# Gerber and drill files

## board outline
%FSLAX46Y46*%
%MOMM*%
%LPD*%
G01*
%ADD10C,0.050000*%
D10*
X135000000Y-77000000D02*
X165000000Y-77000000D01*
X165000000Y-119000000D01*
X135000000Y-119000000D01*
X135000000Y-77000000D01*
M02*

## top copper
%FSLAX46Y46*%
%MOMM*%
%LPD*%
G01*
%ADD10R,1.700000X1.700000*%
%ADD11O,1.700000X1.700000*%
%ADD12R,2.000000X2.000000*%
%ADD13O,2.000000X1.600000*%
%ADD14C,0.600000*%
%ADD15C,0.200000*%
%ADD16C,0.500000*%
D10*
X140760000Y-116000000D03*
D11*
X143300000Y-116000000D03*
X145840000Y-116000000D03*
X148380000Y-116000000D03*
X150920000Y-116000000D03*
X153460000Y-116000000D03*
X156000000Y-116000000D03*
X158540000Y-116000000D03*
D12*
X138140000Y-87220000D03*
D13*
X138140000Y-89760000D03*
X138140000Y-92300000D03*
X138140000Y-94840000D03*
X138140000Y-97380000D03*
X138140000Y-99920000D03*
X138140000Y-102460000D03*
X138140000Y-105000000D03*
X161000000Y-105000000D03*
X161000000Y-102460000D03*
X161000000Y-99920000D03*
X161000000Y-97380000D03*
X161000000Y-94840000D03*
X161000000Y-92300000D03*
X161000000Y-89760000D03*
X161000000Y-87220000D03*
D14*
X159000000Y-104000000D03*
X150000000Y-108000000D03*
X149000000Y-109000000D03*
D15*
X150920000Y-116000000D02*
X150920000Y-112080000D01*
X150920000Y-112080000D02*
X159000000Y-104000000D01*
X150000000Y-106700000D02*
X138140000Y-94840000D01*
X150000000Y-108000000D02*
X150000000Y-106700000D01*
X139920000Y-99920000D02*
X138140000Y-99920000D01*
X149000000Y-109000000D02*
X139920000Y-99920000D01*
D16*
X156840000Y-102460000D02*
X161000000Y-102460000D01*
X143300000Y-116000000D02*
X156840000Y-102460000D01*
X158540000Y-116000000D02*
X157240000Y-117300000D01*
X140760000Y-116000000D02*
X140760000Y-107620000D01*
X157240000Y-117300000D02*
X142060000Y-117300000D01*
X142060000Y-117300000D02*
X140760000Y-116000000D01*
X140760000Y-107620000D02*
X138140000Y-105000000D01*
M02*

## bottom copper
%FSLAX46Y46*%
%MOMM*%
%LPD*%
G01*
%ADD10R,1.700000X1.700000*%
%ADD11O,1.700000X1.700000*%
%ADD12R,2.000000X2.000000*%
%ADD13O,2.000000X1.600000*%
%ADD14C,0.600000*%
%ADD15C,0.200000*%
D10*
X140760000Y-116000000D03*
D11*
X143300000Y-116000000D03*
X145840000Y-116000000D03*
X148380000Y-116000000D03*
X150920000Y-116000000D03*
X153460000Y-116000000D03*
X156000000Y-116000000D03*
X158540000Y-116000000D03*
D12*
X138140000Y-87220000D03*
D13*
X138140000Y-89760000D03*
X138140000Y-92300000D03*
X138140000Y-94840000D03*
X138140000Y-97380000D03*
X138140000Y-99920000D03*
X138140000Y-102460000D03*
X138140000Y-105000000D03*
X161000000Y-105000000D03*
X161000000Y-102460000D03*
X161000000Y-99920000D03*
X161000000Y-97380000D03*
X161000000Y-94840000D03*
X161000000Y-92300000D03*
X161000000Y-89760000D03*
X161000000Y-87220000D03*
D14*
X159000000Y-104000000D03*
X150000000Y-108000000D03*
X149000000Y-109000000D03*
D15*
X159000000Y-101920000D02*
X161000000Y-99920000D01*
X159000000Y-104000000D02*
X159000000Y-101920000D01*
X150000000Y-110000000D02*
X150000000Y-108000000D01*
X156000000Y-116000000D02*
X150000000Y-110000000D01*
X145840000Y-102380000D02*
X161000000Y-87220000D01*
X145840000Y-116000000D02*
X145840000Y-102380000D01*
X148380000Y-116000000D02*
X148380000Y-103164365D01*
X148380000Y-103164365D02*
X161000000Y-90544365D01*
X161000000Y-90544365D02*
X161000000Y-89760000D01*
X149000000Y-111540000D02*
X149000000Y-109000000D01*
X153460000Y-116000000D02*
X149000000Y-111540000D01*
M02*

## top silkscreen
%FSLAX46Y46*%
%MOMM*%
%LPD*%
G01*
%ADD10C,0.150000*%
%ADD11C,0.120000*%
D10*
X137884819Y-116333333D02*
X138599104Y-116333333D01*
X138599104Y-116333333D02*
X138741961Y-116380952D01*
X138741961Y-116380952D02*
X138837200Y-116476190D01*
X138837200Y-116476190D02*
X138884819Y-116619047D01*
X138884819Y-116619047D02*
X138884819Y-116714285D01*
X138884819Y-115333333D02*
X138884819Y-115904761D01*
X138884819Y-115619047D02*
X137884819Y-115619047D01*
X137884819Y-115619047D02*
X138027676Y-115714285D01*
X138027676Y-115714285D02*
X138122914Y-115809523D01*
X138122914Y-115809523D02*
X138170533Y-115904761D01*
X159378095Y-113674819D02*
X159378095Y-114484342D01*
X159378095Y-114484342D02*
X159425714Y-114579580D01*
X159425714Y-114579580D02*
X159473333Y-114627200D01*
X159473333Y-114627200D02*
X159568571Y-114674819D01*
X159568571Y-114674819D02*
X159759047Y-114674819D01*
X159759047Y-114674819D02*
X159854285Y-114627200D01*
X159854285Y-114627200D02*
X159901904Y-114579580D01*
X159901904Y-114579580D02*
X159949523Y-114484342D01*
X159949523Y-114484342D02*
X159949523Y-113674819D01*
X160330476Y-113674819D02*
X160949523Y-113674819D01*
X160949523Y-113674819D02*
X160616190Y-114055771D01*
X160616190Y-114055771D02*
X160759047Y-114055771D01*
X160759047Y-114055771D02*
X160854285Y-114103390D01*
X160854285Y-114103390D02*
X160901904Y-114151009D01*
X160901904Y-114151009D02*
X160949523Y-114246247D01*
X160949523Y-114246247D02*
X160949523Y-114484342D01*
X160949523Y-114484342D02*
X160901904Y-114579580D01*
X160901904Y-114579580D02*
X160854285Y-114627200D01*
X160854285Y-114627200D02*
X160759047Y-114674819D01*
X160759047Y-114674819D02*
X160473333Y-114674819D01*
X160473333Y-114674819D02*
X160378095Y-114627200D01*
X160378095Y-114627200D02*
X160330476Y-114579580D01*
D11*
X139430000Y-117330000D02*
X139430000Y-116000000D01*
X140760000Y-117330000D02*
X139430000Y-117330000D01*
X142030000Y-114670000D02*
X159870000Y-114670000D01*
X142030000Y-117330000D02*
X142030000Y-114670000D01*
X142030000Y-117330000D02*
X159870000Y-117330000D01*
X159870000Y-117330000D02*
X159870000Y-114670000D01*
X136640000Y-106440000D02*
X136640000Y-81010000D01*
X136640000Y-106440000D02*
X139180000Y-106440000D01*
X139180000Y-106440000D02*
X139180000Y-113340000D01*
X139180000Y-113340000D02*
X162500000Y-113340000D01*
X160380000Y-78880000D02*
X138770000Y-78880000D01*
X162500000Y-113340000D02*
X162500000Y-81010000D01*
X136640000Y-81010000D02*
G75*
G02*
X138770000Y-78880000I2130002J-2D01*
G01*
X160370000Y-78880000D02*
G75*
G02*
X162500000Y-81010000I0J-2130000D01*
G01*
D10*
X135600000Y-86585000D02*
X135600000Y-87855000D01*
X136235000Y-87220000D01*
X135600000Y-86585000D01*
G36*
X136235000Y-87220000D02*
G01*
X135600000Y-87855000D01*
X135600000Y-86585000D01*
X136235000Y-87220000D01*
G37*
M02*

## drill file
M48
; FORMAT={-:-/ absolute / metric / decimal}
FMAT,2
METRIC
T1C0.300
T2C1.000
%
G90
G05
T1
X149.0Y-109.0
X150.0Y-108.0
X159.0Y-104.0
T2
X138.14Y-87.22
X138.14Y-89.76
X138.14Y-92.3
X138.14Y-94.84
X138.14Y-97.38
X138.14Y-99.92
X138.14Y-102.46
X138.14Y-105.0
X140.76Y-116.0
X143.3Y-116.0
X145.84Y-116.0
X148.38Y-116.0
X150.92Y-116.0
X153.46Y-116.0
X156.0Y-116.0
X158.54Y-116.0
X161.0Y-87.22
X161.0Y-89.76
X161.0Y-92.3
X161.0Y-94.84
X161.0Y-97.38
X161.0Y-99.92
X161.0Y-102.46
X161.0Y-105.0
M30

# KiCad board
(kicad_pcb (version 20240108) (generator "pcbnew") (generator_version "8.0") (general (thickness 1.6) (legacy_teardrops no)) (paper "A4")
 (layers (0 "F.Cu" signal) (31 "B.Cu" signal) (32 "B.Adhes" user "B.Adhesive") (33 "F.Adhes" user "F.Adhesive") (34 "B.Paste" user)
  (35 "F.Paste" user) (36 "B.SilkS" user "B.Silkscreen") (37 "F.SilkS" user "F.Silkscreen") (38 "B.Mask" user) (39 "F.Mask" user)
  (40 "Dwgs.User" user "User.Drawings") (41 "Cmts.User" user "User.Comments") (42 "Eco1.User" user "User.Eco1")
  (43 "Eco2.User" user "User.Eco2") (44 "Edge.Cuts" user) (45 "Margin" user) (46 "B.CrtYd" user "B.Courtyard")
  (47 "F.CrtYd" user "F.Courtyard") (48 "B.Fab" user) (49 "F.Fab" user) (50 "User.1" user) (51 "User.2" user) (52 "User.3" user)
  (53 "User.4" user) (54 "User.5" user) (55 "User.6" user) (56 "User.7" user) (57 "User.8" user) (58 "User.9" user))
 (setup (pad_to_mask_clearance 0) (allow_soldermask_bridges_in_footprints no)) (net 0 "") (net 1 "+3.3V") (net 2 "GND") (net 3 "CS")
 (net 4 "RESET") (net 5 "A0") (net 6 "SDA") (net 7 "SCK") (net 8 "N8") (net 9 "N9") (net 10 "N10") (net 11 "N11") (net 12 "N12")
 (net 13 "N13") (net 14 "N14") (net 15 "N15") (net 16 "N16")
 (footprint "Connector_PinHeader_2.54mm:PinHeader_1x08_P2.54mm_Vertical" (layer "F.Cu") (at 140.76 116 90)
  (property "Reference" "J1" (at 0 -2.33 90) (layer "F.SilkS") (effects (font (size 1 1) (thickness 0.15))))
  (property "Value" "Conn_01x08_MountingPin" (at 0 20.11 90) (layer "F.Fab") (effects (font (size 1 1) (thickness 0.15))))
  (fp_line (start -1.33 -1.33) (end 0 -1.33) (stroke (width 0.12) (type solid)) (layer "F.SilkS"))
  (fp_line (start -1.33 0) (end -1.33 -1.33) (stroke (width 0.12) (type solid)) (layer "F.SilkS"))
  (fp_line (start 1.33 1.27) (end 1.33 19.11) (stroke (width 0.12) (type solid)) (layer "F.SilkS"))
  (fp_line (start -1.33 1.27) (end 1.33 1.27) (stroke (width 0.12) (type solid)) (layer "F.SilkS"))
  (fp_line (start -1.33 1.27) (end -1.33 19.11) (stroke (width 0.12) (type solid)) (layer "F.SilkS"))
  (fp_line (start -1.33 19.11) (end 1.33 19.11) (stroke (width 0.12) (type solid)) (layer "F.SilkS"))
  (pad "1" thru_hole rect (at 0 0 90) (size 1.7 1.7) (drill 1) (layers "*.Cu" "*.Mask") (remove_unused_layers no) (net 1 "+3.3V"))
  (pad "2" thru_hole oval (at 0 2.54 90) (size 1.7 1.7) (drill 1) (layers "*.Cu" "*.Mask") (remove_unused_layers no) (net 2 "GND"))
  (pad "3" thru_hole oval (at 0 5.08 90) (size 1.7 1.7) (drill 1) (layers "*.Cu" "*.Mask") (remove_unused_layers no) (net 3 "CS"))
  (pad "4" thru_hole oval (at 0 7.62 90) (size 1.7 1.7) (drill 1) (layers "*.Cu" "*.Mask") (remove_unused_layers no) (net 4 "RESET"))
  (pad "5" thru_hole oval (at 0 10.16 90) (size 1.7 1.7) (drill 1) (layers "*.Cu" "*.Mask") (remove_unused_layers no) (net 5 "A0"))
  (pad "6" thru_hole oval (at 0 12.7 90) (size 1.7 1.7) (drill 1) (layers "*.Cu" "*.Mask") (remove_unused_layers no) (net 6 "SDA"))
  (pad "7" thru_hole oval (at 0 15.24 90) (size 1.7 1.7) (drill 1) (layers "*.Cu" "*.Mask") (remove_unused_layers no) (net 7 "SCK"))
  (pad "8" thru_hole oval (at 0 17.78 90) (size 1.7 1.7) (drill 1) (layers "*.Cu" "*.Mask") (remove_unused_layers no) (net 1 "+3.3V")))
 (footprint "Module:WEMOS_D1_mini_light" (layer "F.Cu") (at 138.14 87.22)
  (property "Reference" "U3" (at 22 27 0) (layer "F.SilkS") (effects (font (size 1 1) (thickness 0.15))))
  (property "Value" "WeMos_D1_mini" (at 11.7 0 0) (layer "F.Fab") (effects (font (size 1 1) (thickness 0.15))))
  (fp_line (start -1.5 19.22) (end -1.5 -6.21) (stroke (width 0.12) (type solid)) (layer "F.SilkS"))
  (fp_line (start -1.5 19.22) (end 1.04 19.22) (stroke (width 0.12) (type solid)) (layer "F.SilkS"))
  (fp_line (start 1.04 19.22) (end 1.04 26.12) (stroke (width 0.12) (type solid)) (layer "F.SilkS"))
  (fp_line (start 1.04 26.12) (end 24.36 26.12) (stroke (width 0.12) (type solid)) (layer "F.SilkS"))
  (fp_line (start 22.24 -8.34) (end 0.63 -8.34) (stroke (width 0.12) (type solid)) (layer "F.SilkS"))
  (fp_line (start 24.36 26.12) (end 24.36 -6.21) (stroke (width 0.12) (type solid)) (layer "F.SilkS"))
  (fp_arc (start -1.5 -6.21) (mid -0.876137 -7.716137) (end 0.63 -8.34) (stroke (width 0.12) (type solid)) (layer "F.SilkS"))
  (fp_arc (start 22.23 -8.34) (mid 23.736137 -7.716137) (end 24.36 -6.21) (stroke (width 0.12) (type solid)) (layer "F.SilkS"))
  (fp_poly (pts (xy -2.54 -0.635) (xy -2.54 0.635) (xy -1.905 0)) (stroke (width 0.15) (type solid)) (fill solid) (layer "F.SilkS"))
  (pad "1" thru_hole rect (at 0 0) (size 2 2) (drill 1) (layers "*.Cu" "*.Mask") (remove_unused_layers no) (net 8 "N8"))
  (pad "2" thru_hole oval (at 0 2.54) (size 2 1.6) (drill 1) (layers "*.Cu" "*.Mask") (remove_unused_layers no) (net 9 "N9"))
  (pad "3" thru_hole oval (at 0 5.08) (size 2 1.6) (drill 1) (layers "*.Cu" "*.Mask") (remove_unused_layers no) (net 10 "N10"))
  (pad "4" thru_hole oval (at 0 7.62) (size 2 1.6) (drill 1) (layers "*.Cu" "*.Mask") (remove_unused_layers no) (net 7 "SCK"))
  (pad "5" thru_hole oval (at 0 10.16) (size 2 1.6) (drill 1) (layers "*.Cu" "*.Mask") (remove_unused_layers no) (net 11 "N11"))
  (pad "6" thru_hole oval (at 0 12.7) (size 2 1.6) (drill 1) (layers "*.Cu" "*.Mask") (remove_unused_layers no) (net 6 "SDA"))
  (pad "7" thru_hole oval (at 0 15.24) (size 2 1.6) (drill 1) (layers "*.Cu" "*.Mask") (remove_unused_layers no) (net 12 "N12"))
  (pad "8" thru_hole oval (at 0 17.78) (size 2 1.6) (drill 1) (layers "*.Cu" "*.Mask") (remove_unused_layers no) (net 1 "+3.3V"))
  (pad "9" thru_hole oval (at 22.86 17.78) (size 2 1.6) (drill 1) (layers "*.Cu" "*.Mask") (remove_unused_layers no) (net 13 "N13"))
  (pad "10" thru_hole oval (at 22.86 15.24) (size 2 1.6) (drill 1) (layers "*.Cu" "*.Mask") (remove_unused_layers no) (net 2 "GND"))
  (pad "11" thru_hole oval (at 22.86 12.7) (size 2 1.6) (drill 1) (layers "*.Cu" "*.Mask") (remove_unused_layers no) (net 5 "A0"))
  (pad "12" thru_hole oval (at 22.86 10.16) (size 2 1.6) (drill 1) (layers "*.Cu" "*.Mask") (remove_unused_layers no) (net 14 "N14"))
  (pad "13" thru_hole oval (at 22.86 7.62) (size 2 1.6) (drill 1) (layers "*.Cu" "*.Mask") (remove_unused_layers no) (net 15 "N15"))
  (pad "14" thru_hole oval (at 22.86 5.08) (size 2 1.6) (drill 1) (layers "*.Cu" "*.Mask") (remove_unused_layers no) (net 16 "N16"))
  (pad "15" thru_hole oval (at 22.86 2.54) (size 2 1.6) (drill 1) (layers "*.Cu" "*.Mask") (remove_unused_layers no) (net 4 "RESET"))
  (pad "16" thru_hole oval (at 22.86 0) (size 2 1.6) (drill 1) (layers "*.Cu" "*.Mask") (remove_unused_layers no) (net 3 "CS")))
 (gr_rect (start 135 77) (end 165 119) (stroke (width 0.05) (type default)) (fill none) (layer "Edge.Cuts"))
 (segment (start 150.92 116) (end 150.92 112.08) (width 0.2) (layer "F.Cu") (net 5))
 (segment (start 150.92 112.08) (end 159 104) (width 0.2) (layer "F.Cu") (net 5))
 (via (at 159 104) (size 0.6) (drill 0.3) (layers "F.Cu" "B.Cu") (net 5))
 (segment (start 159 101.92) (end 161 99.92) (width 0.2) (layer "B.Cu") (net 5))
 (segment (start 159 104) (end 159 101.92) (width 0.2) (layer "B.Cu") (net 5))
 (segment (start 150 106.7) (end 138.14 94.84) (width 0.2) (layer "F.Cu") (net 7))
 (segment (start 150 108) (end 150 106.7) (width 0.2) (layer "F.Cu") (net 7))
 (via (at 150 108) (size 0.6) (drill 0.3) (layers "F.Cu" "B.Cu") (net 7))
 (segment (start 150 110) (end 150 108) (width 0.2) (layer "B.Cu") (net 7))
 (segment (start 156 116) (end 150 110) (width 0.2) (layer "B.Cu") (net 7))
 (segment (start 145.84 102.38) (end 161 87.22) (width 0.2) (layer "B.Cu") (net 3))
 (segment (start 145.84 116) (end 145.84 102.38) (width 0.2) (layer "B.Cu") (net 3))
 (segment (start 148.38 116) (end 148.38 103.164365) (width 0.2) (layer "B.Cu") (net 4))
 (segment (start 148.38 103.164365) (end 161 90.544365) (width 0.2) (layer "B.Cu") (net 4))
 (segment (start 161 90.544365) (end 161 89.76) (width 0.2) (layer "B.Cu") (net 4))
 (segment (start 139.92 99.92) (end 138.14 99.92) (width 0.2) (layer "F.Cu") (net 6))
 (segment (start 149 109) (end 139.92 99.92) (width 0.2) (layer "F.Cu") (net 6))
 (via (at 149 109) (size 0.6) (drill 0.3) (layers "F.Cu" "B.Cu") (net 6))
 (segment (start 149 111.54) (end 149 109) (width 0.2) (layer "B.Cu") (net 6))
 (segment (start 153.46 116) (end 149 111.54) (width 0.2) (layer "B.Cu") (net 6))
 (segment (start 156.84 102.46) (end 161 102.46) (width 0.5) (layer "F.Cu") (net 2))
 (segment (start 143.3 116) (end 156.84 102.46) (width 0.5) (layer "F.Cu") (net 2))
 (segment (start 158.54 116) (end 157.24 117.3) (width 0.5) (layer "F.Cu") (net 1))
 (segment (start 140.76 116) (end 140.76 107.62) (width 0.5) (layer "F.Cu") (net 1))
 (segment (start 157.24 117.3) (end 142.06 117.3) (width 0.5) (layer "F.Cu") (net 1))
 (segment (start 142.06 117.3) (end 140.76 116) (width 0.5) (layer "F.Cu") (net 1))
 (segment (start 140.76 107.62) (end 138.14 105) (width 0.5) (layer "F.Cu") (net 1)))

